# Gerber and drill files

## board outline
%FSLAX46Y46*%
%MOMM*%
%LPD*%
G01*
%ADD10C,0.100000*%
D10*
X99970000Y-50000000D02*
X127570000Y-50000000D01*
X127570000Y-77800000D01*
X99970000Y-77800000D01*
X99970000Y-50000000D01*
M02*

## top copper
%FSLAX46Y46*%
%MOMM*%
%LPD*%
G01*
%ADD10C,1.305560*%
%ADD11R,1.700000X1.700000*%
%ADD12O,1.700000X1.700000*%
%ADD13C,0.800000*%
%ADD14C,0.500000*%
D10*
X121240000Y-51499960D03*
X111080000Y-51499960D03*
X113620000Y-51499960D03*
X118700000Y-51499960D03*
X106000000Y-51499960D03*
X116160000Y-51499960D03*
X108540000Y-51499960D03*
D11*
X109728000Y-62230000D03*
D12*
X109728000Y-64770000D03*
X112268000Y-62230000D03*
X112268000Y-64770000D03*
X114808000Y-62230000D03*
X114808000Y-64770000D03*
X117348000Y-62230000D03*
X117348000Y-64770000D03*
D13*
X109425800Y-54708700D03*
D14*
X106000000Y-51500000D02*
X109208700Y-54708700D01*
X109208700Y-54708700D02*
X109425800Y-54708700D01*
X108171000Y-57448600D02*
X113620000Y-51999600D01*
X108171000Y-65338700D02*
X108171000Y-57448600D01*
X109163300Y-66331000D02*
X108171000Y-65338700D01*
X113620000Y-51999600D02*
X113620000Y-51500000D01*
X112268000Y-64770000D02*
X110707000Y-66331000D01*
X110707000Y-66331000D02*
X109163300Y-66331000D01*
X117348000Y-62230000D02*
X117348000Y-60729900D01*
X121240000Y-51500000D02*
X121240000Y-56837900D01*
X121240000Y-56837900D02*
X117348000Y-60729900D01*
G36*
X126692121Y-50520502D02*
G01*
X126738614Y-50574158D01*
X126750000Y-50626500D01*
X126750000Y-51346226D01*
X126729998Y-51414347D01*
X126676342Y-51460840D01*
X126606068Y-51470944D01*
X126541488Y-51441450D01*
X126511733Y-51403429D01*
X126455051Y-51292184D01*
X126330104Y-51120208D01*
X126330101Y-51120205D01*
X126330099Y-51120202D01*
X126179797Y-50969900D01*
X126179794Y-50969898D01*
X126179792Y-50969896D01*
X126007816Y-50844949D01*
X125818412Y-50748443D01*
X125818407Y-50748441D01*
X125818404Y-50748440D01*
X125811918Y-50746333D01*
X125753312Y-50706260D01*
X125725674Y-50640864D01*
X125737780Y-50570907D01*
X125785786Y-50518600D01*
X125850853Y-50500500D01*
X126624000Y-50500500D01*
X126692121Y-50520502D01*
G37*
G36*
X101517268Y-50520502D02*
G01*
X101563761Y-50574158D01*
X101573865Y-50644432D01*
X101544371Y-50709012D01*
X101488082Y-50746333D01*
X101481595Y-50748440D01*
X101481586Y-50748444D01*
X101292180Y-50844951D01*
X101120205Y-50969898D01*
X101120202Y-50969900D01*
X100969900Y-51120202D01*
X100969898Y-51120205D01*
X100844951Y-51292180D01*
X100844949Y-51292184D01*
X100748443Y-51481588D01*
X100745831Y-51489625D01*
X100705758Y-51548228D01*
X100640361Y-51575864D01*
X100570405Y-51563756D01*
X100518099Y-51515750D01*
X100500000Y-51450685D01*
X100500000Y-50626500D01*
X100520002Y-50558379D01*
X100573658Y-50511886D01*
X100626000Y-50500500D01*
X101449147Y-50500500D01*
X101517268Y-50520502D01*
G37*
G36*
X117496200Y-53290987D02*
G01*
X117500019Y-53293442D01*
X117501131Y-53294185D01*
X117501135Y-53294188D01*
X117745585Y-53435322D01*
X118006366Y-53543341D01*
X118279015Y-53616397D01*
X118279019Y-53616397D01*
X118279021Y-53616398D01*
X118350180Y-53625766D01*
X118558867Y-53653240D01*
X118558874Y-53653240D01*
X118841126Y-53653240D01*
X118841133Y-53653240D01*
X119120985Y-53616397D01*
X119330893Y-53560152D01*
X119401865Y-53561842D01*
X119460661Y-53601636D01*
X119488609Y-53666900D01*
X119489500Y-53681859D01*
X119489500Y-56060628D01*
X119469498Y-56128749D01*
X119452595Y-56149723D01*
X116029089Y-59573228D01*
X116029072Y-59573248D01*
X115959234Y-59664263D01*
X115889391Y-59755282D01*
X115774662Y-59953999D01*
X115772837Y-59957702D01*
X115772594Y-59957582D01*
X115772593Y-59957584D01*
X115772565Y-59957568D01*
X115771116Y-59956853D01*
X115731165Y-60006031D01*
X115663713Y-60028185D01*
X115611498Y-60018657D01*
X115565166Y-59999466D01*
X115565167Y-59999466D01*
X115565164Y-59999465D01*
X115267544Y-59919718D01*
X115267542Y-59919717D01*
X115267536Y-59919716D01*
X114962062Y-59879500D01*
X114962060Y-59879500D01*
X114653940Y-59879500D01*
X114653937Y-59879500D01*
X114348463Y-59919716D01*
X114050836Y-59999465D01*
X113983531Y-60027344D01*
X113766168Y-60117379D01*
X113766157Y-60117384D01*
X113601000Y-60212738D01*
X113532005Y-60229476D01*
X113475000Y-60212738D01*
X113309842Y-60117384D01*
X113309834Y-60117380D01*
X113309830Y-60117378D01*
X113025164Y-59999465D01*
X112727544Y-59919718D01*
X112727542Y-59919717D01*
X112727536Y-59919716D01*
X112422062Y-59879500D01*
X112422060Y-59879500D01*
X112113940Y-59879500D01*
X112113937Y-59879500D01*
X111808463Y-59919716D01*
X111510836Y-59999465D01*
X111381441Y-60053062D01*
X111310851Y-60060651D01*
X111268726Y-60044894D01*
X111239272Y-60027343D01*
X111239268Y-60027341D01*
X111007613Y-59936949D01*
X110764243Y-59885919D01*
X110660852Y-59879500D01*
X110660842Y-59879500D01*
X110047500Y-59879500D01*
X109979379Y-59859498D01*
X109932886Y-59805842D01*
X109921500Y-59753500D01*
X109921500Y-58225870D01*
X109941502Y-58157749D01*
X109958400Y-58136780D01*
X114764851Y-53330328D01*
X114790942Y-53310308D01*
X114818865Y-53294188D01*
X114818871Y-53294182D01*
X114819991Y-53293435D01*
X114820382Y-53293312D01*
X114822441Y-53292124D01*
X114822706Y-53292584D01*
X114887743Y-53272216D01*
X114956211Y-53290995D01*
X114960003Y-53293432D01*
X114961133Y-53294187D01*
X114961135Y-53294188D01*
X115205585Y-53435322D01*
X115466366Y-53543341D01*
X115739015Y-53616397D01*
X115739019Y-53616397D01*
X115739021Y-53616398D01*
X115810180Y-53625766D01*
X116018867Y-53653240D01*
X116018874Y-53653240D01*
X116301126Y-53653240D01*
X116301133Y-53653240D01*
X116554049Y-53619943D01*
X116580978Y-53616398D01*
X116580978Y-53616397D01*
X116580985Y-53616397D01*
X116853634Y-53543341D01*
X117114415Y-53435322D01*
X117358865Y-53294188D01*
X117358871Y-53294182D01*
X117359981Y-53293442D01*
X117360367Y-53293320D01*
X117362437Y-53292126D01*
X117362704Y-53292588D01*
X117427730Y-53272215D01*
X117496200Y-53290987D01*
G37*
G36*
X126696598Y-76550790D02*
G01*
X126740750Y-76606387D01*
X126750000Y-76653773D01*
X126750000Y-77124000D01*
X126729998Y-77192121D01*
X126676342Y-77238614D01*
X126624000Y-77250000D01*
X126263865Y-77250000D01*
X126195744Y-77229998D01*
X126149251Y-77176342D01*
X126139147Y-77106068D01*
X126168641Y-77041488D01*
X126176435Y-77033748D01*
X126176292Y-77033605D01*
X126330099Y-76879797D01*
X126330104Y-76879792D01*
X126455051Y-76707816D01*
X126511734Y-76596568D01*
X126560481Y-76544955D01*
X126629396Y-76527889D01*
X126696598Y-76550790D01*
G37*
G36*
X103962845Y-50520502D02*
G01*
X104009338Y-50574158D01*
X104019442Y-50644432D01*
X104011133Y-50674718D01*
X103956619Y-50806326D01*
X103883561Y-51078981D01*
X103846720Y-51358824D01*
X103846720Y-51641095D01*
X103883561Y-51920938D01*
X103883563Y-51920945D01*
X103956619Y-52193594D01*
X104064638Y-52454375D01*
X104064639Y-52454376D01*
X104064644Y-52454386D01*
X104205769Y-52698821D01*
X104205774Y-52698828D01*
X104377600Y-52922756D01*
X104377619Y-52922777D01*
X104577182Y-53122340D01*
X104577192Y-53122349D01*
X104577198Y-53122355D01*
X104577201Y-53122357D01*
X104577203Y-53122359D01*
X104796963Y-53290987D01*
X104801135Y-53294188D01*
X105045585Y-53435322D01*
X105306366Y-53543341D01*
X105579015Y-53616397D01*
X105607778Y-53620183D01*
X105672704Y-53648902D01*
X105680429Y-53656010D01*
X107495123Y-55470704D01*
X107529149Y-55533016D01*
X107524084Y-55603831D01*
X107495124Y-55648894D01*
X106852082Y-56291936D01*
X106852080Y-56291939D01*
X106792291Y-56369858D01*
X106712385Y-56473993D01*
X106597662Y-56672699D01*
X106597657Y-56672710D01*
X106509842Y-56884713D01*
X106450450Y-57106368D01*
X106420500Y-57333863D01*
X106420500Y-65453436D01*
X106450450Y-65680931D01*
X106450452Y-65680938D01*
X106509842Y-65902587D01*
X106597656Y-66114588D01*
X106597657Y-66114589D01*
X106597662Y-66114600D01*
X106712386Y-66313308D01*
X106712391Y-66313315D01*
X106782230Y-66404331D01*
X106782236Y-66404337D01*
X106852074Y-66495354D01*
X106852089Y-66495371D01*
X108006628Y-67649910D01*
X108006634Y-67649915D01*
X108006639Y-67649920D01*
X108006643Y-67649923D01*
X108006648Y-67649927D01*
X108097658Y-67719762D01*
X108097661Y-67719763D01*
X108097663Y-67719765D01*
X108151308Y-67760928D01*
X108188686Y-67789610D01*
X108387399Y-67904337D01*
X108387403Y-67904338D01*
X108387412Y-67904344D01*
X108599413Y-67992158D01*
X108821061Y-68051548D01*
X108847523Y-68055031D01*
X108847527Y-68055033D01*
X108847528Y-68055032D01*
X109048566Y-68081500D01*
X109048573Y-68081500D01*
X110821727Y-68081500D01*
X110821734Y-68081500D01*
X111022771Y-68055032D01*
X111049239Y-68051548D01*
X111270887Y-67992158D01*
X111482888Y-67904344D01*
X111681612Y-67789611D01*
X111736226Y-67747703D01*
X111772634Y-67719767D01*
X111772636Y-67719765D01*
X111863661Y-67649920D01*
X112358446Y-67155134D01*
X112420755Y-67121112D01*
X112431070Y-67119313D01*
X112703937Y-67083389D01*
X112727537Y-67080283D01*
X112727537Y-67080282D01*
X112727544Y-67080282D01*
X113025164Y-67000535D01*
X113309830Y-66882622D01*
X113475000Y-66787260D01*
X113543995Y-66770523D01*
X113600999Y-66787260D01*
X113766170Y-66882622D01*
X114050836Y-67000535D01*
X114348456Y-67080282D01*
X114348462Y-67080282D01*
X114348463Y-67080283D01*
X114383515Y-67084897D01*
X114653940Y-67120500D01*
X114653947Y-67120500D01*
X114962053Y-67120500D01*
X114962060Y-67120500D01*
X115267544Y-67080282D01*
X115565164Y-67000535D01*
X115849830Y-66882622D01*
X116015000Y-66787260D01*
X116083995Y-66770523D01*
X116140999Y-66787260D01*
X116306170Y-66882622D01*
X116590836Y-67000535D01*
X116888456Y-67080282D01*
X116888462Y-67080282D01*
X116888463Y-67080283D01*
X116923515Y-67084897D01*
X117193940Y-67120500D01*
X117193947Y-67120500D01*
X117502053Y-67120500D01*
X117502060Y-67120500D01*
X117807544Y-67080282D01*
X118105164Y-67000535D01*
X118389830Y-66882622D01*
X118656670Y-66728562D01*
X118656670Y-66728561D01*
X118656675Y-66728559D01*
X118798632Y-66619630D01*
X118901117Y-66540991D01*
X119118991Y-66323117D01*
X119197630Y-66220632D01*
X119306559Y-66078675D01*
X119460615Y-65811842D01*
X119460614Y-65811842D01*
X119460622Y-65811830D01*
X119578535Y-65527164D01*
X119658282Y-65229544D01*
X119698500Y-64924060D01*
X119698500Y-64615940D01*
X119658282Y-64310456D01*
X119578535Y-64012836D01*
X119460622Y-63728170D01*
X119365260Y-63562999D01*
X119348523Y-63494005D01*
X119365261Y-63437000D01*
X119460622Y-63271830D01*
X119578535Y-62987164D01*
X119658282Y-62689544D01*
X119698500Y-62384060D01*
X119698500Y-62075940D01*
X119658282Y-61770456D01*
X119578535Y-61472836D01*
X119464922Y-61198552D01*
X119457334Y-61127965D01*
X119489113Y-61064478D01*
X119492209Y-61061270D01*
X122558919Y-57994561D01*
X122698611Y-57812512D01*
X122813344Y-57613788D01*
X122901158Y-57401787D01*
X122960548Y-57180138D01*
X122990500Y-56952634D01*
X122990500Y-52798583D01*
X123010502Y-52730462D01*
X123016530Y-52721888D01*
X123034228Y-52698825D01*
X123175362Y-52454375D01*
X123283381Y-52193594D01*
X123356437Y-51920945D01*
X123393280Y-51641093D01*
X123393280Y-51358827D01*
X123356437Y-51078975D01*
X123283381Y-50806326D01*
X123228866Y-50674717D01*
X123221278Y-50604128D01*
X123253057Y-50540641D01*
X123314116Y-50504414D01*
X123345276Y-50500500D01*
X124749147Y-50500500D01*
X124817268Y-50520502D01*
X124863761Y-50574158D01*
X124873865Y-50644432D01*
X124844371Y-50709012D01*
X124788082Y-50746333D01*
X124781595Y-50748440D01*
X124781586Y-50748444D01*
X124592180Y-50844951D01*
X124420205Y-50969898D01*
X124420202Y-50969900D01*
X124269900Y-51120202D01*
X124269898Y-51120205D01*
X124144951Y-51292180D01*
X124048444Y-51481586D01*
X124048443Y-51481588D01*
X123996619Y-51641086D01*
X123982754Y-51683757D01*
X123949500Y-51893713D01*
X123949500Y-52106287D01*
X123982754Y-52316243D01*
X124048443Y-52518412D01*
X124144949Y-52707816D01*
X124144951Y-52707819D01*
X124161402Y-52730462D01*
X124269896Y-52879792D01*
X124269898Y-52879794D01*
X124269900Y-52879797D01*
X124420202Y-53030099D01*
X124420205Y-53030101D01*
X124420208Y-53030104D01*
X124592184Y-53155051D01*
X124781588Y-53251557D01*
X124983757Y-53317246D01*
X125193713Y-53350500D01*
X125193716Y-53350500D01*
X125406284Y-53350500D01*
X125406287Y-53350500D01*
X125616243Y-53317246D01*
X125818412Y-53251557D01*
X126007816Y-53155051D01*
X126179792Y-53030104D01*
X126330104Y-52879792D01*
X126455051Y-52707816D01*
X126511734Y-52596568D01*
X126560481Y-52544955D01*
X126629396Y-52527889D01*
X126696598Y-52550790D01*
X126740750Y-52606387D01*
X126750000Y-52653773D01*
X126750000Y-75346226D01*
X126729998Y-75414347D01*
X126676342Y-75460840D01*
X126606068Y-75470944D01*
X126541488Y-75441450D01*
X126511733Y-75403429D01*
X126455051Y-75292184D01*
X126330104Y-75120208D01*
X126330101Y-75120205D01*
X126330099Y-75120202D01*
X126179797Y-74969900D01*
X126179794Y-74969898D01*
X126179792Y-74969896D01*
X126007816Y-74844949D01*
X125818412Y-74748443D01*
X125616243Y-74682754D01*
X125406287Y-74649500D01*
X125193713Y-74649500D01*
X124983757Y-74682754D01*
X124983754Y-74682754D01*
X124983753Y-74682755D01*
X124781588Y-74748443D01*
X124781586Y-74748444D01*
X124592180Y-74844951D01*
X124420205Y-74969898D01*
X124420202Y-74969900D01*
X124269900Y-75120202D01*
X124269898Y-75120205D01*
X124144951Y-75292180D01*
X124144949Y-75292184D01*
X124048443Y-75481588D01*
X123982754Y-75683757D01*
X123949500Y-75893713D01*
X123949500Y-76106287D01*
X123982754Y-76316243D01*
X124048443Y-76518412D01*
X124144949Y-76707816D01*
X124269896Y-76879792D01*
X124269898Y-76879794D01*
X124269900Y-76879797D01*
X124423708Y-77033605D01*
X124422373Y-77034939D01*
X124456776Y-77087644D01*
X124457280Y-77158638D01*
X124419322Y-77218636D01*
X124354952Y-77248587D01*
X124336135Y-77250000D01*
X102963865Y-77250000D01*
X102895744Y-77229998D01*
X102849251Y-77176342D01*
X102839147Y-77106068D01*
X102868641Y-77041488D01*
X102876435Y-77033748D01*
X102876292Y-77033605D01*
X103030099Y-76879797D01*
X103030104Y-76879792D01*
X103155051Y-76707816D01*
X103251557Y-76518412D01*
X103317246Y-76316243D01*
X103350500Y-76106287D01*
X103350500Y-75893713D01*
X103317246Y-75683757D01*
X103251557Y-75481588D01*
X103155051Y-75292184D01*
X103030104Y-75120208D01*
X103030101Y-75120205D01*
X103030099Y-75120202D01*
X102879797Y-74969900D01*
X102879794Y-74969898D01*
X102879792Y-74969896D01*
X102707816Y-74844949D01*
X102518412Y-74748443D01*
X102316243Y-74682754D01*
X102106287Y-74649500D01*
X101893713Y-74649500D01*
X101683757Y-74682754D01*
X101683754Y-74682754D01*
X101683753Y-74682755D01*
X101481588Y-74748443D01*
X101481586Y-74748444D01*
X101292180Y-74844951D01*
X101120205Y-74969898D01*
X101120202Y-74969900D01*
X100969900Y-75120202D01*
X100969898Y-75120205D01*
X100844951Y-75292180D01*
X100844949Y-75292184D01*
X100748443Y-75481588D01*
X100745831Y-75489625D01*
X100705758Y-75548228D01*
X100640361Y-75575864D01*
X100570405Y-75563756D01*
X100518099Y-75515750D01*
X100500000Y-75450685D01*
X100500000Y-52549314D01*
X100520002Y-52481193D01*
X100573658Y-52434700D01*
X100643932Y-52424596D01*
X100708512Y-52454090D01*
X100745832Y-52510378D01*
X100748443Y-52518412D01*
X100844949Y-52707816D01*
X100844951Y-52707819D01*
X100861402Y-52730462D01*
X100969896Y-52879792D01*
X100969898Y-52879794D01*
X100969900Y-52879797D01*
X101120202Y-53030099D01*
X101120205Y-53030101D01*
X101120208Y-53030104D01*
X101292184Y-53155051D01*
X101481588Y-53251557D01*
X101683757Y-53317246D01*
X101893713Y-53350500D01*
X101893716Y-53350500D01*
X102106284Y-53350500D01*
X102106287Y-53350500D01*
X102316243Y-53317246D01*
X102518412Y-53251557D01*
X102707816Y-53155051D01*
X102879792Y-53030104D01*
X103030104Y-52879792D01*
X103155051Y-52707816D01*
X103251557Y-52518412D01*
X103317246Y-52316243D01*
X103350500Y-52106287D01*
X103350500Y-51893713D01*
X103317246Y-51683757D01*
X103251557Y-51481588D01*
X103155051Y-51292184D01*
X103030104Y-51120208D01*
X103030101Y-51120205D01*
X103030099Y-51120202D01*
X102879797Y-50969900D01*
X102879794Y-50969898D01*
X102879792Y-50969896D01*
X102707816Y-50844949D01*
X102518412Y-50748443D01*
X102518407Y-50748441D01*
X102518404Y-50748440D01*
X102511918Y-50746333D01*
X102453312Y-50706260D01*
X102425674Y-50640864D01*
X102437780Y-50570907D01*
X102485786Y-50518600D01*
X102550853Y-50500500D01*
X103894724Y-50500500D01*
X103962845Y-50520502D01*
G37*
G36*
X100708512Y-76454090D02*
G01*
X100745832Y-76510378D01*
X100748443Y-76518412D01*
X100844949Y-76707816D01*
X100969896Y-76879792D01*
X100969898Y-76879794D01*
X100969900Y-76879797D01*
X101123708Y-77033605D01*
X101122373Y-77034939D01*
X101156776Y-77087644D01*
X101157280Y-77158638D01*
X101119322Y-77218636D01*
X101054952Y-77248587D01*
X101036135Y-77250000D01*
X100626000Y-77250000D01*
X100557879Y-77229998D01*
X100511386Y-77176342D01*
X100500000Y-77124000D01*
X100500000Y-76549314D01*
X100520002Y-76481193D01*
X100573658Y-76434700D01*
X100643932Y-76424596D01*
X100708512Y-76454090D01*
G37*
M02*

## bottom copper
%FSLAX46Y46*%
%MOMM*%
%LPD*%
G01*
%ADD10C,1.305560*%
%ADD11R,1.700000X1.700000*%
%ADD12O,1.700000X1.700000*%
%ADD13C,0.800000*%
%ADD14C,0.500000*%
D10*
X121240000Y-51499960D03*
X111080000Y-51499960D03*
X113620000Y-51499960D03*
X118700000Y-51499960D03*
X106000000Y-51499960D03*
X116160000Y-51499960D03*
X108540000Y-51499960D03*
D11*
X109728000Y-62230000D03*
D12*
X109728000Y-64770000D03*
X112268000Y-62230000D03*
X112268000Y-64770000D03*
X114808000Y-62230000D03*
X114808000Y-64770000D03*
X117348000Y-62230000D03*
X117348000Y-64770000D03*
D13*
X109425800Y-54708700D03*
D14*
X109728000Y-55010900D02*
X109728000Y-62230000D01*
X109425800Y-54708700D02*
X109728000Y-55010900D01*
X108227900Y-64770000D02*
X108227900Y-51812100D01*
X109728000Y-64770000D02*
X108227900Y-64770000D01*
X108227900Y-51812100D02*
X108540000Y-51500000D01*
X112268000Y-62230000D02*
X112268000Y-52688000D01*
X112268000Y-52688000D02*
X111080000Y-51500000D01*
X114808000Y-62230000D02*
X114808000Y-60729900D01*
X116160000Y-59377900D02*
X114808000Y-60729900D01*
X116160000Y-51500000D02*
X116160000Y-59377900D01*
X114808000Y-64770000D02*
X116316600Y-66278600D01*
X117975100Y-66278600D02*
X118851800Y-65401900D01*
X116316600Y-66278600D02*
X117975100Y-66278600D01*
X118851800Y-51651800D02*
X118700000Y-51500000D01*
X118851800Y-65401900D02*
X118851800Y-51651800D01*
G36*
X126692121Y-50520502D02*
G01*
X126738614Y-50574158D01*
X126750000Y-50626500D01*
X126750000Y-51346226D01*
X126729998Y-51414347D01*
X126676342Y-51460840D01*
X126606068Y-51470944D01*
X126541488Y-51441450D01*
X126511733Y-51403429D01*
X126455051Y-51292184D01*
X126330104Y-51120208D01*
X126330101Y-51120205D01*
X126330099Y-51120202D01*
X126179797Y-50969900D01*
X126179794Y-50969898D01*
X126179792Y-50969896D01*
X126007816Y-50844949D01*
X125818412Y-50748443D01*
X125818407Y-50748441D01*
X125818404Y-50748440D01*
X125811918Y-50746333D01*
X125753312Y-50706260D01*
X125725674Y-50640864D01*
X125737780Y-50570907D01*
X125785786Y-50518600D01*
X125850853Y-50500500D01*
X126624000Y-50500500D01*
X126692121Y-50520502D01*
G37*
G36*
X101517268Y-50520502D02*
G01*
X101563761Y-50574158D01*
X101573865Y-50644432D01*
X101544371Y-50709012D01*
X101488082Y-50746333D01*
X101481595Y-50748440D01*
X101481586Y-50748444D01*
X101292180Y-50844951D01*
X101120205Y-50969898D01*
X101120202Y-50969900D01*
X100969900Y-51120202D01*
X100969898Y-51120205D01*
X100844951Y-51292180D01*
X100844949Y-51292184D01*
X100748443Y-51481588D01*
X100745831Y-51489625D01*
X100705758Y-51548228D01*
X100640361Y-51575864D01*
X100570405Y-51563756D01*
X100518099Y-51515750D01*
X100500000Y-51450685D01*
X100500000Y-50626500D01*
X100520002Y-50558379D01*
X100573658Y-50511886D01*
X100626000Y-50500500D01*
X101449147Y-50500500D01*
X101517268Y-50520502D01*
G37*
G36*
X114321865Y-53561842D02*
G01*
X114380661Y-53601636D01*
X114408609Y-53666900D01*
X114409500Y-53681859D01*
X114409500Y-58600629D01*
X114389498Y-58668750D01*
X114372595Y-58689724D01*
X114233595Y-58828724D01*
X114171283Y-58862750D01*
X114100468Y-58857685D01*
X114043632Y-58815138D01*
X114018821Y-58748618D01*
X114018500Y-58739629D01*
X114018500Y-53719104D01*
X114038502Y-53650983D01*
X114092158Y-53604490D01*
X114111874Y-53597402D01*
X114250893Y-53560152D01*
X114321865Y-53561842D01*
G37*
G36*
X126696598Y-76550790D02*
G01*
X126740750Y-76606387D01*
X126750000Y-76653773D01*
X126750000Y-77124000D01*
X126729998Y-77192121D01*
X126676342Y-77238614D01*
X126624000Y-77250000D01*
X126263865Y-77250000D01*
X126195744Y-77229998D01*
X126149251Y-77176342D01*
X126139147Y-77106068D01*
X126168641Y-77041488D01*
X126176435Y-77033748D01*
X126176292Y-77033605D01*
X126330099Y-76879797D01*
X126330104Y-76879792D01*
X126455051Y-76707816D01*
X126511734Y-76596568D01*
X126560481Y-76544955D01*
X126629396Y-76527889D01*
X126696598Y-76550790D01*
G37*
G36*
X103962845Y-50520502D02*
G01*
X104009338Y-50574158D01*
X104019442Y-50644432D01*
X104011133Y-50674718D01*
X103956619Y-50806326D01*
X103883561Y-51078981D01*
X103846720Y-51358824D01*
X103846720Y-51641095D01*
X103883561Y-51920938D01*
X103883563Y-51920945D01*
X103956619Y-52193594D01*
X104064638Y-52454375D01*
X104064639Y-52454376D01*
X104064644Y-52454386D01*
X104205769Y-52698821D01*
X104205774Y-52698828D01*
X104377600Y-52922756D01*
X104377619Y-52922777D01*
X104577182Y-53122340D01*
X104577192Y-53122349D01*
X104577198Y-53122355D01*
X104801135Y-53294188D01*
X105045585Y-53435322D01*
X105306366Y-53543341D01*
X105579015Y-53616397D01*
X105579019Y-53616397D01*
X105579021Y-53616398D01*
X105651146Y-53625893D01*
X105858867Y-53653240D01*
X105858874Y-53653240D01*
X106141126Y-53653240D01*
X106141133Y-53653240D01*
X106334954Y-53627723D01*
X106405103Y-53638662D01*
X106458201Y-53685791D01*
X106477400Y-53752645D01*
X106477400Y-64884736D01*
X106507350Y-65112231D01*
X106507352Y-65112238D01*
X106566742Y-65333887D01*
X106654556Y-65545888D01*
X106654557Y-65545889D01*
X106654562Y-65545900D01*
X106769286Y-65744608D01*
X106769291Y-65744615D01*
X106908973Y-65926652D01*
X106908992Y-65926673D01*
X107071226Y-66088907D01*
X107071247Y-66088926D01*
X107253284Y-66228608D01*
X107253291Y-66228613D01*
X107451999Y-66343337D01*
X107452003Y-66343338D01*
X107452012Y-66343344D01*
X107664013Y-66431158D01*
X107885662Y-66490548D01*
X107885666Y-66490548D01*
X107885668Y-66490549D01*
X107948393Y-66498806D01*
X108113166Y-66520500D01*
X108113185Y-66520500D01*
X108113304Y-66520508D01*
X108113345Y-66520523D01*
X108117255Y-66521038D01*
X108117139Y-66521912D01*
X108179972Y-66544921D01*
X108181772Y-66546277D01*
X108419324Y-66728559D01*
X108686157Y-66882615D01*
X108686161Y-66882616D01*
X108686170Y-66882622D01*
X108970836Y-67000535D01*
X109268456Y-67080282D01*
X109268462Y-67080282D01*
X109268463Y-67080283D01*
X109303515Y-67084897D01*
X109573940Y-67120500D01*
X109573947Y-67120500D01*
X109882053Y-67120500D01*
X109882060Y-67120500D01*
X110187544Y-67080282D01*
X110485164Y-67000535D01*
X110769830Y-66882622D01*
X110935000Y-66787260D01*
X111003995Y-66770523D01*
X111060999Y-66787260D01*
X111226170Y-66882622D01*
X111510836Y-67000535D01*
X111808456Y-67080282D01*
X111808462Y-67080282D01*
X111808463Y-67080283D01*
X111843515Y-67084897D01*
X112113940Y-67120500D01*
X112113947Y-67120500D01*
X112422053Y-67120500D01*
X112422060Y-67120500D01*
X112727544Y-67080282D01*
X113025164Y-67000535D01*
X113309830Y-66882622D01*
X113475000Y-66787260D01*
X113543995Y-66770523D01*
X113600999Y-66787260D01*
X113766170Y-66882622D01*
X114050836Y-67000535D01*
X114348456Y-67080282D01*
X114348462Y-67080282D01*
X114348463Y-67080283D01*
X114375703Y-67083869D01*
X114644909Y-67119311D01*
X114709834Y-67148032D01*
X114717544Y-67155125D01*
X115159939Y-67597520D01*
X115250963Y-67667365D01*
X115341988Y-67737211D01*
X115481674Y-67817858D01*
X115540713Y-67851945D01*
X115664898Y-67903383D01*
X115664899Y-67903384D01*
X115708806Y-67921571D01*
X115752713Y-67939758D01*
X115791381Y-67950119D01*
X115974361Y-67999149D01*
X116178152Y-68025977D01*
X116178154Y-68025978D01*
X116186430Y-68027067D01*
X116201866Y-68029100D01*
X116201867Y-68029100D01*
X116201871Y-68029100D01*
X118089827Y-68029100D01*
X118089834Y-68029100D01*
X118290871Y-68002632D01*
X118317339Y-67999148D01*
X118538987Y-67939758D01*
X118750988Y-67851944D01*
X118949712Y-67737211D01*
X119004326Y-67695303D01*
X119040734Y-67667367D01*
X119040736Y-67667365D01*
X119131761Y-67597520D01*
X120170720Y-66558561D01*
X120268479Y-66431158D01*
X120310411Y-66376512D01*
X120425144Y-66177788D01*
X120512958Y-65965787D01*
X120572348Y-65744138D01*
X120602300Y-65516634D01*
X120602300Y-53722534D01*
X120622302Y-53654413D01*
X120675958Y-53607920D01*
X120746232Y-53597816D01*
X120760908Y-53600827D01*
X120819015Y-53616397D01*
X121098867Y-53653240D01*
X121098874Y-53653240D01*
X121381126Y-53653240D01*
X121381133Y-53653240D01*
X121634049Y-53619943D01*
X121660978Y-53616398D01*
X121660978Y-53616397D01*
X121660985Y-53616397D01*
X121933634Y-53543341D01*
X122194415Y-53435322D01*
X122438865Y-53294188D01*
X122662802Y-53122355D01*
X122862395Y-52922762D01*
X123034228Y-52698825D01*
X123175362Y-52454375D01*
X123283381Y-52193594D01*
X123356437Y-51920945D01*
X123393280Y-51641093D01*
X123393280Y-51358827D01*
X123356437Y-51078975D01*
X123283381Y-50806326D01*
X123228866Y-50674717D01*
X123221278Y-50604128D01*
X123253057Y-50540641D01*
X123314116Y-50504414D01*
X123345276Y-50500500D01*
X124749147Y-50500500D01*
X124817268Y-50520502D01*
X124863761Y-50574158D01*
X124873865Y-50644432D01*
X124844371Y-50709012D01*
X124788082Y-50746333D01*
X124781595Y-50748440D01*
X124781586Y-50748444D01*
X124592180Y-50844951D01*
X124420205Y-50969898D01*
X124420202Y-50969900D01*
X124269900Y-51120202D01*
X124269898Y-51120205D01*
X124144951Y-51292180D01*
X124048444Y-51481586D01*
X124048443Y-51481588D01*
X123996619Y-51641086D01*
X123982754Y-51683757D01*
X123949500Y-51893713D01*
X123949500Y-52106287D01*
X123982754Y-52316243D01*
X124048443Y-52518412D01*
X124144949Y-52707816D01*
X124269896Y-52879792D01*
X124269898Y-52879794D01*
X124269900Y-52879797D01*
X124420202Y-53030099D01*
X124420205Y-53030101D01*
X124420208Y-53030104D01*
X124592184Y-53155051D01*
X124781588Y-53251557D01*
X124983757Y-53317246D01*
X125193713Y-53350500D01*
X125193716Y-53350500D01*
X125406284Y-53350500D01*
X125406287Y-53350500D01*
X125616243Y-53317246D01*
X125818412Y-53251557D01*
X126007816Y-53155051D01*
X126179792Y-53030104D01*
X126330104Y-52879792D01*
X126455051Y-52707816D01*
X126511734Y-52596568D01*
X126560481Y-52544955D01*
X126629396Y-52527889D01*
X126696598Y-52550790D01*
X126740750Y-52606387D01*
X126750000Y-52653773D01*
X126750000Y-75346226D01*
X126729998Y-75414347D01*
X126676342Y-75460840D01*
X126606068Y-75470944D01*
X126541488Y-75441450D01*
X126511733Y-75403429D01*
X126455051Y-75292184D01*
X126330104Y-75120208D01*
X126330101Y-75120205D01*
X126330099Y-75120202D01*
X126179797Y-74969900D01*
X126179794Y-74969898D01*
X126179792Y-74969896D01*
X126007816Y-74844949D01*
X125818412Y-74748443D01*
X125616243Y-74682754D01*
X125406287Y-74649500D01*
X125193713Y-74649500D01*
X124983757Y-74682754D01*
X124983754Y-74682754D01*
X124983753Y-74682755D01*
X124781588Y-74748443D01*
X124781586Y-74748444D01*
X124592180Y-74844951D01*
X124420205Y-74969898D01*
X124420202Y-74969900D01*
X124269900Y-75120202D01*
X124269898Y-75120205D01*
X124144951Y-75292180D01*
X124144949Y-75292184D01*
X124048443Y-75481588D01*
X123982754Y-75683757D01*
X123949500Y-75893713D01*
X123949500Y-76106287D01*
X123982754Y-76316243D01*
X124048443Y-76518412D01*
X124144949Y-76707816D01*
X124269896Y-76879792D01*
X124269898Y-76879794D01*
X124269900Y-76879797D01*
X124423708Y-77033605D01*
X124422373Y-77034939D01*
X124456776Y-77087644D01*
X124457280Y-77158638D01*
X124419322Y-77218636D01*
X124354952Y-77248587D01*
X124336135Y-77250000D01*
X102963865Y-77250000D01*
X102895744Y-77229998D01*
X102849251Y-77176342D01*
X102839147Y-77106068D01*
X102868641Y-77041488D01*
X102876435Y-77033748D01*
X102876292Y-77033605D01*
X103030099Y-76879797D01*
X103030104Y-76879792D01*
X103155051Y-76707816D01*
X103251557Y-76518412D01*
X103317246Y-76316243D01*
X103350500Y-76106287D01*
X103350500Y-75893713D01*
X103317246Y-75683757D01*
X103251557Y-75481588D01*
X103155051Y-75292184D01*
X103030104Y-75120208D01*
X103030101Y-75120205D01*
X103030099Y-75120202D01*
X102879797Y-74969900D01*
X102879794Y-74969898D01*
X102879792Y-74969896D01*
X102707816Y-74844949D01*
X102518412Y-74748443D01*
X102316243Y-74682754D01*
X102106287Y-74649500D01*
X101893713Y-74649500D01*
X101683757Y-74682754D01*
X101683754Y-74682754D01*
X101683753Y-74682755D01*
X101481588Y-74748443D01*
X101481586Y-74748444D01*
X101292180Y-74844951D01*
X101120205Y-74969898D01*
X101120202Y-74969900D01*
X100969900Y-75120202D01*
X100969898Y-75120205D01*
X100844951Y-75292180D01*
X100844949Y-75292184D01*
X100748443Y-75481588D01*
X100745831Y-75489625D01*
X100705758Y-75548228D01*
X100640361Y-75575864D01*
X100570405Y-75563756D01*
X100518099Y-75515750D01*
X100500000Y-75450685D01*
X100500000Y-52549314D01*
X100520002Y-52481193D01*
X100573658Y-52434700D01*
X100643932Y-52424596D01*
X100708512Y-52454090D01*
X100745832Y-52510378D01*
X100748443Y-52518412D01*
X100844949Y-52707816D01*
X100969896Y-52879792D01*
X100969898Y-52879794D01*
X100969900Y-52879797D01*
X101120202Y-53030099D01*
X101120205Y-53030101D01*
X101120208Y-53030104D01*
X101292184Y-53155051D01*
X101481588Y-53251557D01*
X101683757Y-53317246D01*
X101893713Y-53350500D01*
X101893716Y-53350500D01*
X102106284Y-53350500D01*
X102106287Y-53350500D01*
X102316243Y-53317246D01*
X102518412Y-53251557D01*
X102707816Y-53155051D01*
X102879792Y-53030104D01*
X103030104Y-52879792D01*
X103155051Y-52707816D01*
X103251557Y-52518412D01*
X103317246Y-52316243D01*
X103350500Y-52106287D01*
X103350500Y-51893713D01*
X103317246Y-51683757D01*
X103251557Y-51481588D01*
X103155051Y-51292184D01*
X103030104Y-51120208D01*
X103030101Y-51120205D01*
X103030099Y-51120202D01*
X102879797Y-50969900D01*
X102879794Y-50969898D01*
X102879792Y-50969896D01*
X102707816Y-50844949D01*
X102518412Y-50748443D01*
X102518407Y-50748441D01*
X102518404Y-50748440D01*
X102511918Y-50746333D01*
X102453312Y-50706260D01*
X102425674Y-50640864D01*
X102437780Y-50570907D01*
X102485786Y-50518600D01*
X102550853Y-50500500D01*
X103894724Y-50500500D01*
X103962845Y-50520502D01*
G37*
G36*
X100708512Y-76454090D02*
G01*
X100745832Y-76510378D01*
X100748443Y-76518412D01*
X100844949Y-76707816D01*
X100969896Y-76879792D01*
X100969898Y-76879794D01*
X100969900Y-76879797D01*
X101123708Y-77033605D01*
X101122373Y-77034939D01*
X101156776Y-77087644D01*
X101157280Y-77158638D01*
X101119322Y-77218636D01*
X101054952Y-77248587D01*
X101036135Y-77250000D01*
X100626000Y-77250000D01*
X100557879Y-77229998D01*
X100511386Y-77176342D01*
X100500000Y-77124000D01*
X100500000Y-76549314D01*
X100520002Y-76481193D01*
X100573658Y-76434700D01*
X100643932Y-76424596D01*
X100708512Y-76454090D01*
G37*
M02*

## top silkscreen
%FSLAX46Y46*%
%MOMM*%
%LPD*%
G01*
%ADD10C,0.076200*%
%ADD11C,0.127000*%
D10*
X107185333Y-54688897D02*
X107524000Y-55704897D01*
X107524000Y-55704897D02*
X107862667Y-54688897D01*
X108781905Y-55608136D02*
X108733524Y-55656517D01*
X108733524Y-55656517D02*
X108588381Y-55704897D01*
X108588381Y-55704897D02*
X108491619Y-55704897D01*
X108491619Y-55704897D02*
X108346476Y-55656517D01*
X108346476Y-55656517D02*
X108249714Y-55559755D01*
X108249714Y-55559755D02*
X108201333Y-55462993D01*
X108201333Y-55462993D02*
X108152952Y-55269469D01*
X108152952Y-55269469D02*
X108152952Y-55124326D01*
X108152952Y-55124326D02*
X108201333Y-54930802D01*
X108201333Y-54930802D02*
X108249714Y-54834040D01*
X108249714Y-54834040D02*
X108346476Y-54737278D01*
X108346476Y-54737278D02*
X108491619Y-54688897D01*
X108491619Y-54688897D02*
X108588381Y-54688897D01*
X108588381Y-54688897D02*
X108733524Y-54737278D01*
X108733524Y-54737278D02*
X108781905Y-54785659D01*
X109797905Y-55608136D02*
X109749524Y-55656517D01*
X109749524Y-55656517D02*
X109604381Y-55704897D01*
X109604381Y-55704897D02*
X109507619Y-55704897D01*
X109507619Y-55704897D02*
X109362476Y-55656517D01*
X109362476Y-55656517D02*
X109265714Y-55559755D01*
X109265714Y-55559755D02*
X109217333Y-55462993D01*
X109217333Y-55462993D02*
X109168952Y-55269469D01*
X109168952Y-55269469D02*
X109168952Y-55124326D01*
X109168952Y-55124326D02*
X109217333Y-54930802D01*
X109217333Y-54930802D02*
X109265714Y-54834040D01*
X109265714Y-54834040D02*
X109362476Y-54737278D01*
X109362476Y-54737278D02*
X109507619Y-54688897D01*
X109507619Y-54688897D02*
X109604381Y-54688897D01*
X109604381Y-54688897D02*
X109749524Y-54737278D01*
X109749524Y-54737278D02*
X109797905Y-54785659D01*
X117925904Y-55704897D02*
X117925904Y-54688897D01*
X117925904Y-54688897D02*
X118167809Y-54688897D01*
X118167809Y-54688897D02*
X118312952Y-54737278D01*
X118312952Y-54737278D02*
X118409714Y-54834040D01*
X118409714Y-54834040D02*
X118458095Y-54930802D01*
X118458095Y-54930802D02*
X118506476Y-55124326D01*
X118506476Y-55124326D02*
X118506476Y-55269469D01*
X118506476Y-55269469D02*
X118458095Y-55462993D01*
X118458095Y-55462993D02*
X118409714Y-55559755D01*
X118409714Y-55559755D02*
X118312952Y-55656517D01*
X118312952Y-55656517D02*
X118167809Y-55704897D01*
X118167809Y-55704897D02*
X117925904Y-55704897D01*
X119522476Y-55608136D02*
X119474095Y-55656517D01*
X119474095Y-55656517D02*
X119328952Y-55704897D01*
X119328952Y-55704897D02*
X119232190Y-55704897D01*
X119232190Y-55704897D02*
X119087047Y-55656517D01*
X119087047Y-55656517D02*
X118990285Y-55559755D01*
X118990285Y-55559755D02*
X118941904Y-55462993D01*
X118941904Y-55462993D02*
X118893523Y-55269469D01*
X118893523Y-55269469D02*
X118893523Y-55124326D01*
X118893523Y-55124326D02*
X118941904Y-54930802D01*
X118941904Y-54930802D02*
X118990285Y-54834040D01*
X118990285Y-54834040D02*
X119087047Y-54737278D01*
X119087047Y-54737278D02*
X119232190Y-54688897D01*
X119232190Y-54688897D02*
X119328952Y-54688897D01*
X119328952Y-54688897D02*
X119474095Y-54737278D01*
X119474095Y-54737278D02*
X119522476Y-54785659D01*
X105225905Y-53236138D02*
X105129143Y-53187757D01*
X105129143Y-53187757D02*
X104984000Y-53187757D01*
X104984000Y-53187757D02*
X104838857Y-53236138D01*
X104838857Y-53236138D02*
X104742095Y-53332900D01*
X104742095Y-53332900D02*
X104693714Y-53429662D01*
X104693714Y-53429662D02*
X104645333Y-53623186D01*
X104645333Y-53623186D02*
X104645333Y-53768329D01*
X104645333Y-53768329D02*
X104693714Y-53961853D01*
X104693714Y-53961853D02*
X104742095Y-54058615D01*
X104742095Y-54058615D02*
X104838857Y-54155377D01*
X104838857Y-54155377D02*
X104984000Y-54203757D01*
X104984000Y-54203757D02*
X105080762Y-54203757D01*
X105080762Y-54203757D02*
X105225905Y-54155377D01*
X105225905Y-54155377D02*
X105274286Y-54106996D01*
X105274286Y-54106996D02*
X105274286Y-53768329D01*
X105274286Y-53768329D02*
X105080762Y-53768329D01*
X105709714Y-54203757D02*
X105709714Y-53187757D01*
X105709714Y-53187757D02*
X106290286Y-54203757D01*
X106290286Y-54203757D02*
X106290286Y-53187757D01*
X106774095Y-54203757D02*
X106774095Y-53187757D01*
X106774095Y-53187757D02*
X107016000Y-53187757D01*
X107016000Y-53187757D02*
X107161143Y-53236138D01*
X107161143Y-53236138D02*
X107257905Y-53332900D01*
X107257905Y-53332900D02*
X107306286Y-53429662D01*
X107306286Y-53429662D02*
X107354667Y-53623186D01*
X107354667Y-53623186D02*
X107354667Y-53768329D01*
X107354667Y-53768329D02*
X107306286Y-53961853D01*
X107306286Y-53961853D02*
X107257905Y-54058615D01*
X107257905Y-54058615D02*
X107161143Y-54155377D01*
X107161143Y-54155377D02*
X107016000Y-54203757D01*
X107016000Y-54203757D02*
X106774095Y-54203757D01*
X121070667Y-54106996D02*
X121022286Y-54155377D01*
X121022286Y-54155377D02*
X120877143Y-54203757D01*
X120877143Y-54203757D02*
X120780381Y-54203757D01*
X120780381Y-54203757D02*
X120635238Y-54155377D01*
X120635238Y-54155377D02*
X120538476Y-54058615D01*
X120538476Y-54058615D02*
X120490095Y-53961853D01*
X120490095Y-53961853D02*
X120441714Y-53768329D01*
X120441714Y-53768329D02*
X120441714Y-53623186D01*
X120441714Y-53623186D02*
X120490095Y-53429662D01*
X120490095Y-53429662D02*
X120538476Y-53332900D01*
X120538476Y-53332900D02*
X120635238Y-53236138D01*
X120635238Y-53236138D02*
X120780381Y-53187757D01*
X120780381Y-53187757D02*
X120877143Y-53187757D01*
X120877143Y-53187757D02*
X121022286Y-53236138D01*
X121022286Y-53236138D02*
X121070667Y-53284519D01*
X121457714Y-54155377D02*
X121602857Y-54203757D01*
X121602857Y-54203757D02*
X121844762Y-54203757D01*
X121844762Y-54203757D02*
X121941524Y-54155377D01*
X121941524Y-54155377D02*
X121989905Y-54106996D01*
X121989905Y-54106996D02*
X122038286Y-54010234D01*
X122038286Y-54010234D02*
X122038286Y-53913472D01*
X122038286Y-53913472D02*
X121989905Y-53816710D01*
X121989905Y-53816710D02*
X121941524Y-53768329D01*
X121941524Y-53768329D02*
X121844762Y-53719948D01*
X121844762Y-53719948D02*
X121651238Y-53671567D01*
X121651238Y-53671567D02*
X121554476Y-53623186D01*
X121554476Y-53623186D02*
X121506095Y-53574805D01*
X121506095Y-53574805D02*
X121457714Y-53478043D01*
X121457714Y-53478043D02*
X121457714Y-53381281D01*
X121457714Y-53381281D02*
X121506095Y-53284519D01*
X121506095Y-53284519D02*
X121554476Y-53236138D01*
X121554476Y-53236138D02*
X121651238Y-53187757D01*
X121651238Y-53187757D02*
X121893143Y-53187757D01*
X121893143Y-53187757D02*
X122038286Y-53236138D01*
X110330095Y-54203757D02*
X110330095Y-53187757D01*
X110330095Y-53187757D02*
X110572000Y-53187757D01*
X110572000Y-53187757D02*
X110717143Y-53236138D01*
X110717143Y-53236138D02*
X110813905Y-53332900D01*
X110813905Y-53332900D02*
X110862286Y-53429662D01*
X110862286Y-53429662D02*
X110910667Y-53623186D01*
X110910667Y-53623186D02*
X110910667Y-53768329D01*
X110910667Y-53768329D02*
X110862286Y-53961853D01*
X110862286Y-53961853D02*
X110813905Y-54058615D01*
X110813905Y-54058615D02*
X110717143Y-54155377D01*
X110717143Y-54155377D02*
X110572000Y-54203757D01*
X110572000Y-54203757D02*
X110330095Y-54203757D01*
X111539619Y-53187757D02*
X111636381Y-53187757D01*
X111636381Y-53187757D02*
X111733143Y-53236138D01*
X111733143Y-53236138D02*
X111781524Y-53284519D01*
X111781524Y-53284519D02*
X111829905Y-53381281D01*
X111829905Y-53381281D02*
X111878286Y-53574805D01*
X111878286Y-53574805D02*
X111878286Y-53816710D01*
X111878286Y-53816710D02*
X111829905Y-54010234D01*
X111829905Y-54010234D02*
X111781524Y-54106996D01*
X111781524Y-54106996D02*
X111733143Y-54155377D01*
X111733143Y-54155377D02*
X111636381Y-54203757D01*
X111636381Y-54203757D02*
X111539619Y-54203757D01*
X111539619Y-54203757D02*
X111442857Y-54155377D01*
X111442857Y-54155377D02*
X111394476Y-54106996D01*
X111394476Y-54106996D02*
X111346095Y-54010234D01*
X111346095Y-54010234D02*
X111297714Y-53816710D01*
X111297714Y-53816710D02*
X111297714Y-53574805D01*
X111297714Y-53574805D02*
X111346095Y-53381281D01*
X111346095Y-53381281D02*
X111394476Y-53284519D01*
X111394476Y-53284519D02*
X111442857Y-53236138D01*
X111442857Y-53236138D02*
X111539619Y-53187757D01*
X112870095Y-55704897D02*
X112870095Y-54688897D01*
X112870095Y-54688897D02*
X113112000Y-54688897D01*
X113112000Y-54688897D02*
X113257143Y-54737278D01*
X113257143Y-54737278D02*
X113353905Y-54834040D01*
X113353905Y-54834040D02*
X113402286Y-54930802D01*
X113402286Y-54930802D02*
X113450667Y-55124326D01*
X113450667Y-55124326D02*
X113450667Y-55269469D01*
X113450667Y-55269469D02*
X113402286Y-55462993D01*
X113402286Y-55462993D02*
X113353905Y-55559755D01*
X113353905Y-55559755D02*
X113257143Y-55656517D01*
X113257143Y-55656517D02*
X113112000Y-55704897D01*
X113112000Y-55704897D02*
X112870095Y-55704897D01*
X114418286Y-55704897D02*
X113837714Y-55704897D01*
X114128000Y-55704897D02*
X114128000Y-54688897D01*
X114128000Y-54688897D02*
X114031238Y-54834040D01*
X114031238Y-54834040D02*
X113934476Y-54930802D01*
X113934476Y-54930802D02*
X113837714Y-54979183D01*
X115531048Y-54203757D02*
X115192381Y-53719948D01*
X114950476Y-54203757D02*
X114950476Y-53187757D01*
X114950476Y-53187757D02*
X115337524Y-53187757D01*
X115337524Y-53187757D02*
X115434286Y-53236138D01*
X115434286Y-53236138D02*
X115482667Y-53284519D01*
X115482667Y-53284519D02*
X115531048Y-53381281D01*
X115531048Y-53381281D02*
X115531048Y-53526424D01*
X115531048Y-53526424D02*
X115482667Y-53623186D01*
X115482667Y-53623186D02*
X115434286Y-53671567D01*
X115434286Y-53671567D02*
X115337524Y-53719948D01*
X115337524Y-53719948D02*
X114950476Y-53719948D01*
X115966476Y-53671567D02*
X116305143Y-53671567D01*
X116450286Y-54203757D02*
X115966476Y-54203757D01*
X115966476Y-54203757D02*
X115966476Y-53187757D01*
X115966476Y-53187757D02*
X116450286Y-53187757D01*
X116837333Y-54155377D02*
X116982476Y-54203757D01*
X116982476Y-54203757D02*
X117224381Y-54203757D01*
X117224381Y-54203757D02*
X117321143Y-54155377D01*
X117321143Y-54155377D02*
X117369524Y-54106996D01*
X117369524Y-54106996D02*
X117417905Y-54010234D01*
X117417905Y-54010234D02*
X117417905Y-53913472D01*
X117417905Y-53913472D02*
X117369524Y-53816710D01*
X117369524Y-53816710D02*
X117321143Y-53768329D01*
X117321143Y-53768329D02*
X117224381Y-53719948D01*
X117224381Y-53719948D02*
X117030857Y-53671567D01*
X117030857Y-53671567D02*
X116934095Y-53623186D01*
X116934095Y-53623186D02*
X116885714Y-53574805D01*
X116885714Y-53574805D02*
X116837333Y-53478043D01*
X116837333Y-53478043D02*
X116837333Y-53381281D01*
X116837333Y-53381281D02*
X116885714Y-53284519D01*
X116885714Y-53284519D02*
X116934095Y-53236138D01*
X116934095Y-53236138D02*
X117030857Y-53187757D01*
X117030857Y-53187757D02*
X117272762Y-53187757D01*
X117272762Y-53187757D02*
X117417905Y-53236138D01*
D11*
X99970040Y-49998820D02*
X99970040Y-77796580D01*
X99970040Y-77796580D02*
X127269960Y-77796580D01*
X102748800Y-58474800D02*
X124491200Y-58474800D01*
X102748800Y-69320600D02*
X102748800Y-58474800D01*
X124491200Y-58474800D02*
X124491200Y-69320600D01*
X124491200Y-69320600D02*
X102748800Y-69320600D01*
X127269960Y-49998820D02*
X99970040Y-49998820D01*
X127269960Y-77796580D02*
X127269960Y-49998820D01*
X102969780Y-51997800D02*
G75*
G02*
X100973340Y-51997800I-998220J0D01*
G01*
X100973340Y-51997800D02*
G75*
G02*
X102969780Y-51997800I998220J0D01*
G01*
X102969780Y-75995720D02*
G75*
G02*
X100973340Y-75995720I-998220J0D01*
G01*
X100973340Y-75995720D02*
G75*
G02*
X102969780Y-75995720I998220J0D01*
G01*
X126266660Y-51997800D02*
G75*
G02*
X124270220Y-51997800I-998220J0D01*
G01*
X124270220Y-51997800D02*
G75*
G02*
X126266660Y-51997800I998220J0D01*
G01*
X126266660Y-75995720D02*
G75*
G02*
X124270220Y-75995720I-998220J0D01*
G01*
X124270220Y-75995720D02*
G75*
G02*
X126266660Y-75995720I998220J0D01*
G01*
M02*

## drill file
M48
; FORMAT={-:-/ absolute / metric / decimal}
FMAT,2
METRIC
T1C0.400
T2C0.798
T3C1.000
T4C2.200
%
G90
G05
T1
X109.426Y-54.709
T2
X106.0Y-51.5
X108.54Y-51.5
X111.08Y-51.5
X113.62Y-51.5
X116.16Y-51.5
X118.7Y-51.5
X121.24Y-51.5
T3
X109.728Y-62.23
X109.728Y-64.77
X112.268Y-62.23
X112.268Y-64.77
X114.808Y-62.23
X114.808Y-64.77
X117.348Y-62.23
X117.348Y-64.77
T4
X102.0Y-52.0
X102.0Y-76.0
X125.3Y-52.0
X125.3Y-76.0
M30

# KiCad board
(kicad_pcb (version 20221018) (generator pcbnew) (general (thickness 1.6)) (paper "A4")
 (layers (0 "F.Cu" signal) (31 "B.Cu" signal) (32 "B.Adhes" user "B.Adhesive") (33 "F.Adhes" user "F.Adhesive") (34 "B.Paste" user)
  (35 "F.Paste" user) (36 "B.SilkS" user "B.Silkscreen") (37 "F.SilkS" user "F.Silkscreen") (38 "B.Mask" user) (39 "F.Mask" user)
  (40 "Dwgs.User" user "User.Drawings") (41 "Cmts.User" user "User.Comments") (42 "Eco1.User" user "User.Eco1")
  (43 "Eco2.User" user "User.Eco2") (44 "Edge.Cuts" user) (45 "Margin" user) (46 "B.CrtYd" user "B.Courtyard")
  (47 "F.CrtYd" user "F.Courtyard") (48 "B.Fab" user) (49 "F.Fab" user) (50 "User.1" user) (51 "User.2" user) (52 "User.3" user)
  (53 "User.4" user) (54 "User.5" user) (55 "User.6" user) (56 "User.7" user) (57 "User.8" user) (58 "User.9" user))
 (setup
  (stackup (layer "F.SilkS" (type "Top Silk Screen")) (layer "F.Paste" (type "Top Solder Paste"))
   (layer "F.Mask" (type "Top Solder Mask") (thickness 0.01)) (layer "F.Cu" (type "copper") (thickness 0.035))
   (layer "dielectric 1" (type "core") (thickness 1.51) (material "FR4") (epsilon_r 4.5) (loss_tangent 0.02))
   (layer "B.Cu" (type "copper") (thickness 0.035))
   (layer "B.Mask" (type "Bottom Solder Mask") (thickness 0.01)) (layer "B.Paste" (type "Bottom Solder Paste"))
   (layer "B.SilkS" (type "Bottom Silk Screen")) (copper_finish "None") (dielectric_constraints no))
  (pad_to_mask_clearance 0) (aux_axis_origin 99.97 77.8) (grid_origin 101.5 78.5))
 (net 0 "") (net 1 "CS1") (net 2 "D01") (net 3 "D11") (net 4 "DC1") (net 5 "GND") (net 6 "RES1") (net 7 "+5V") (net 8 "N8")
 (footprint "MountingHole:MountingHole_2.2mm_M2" (layer "F.Cu") (at 125.3 52)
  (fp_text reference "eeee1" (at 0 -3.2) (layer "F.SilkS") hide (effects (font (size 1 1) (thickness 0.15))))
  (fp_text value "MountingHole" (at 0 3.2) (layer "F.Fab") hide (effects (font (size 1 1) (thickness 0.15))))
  (pad "" np_thru_hole circle (at 0 0) (size 2.2 2.2) (drill 2.2) (layers "*.Cu" "*.Mask")))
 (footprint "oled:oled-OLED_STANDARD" (layer "F.Cu") (at 113.62 63.8977)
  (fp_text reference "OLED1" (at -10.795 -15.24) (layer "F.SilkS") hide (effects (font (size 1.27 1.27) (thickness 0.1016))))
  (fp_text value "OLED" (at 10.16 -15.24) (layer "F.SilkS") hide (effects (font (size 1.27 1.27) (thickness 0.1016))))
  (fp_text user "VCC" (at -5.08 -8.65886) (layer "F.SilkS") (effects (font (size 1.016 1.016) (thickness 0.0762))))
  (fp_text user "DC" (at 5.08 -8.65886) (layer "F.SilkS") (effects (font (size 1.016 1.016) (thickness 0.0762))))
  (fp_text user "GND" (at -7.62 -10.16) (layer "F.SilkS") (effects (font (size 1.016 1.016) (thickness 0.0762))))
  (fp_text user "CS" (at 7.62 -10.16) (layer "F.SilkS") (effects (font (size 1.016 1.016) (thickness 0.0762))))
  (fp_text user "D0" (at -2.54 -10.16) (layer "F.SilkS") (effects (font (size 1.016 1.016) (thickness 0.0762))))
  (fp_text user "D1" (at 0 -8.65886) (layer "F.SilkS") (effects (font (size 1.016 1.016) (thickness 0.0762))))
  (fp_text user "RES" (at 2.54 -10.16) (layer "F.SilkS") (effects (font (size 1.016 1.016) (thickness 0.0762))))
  (fp_line (start -13.64996 -13.89888) (end -13.64996 13.89888) (stroke (width 0.127) (type solid)) (layer "F.SilkS"))
  (fp_line (start -13.64996 13.89888) (end 13.64996 13.89888) (stroke (width 0.127) (type solid)) (layer "F.SilkS"))
  (fp_line (start -10.8712 -5.4229) (end 10.8712 -5.4229) (stroke (width 0.127) (type solid)) (layer "F.SilkS"))
  (fp_line (start -10.8712 5.4229) (end -10.8712 -5.4229) (stroke (width 0.127) (type solid)) (layer "F.SilkS"))
  (fp_line (start 10.8712 -5.4229) (end 10.8712 5.4229) (stroke (width 0.127) (type solid)) (layer "F.SilkS"))
  (fp_line (start 10.8712 5.4229) (end -10.8712 5.4229) (stroke (width 0.127) (type solid)) (layer "F.SilkS"))
  (fp_line (start 13.64996 -13.89888) (end -13.64996 -13.89888) (stroke (width 0.127) (type solid)) (layer "F.SilkS"))
  (fp_line (start 13.64996 13.89888) (end 13.64996 -13.89888) (stroke (width 0.127) (type solid)) (layer "F.SilkS"))
  (fp_circle (center -11.64844 -11.8999) (end -11.64844 -12.89812) (stroke (width 0.127) (type solid)) (fill none) (layer "F.SilkS"))
  (fp_circle (center -11.64844 12.09802) (end -11.64844 11.0998) (stroke (width 0.127) (type solid)) (fill none) (layer "F.SilkS"))
  (fp_circle (center 11.64844 -11.8999) (end 11.64844 -12.89812) (stroke (width 0.127) (type solid)) (fill none) (layer "F.SilkS"))
  (fp_circle (center 11.64844 12.09802) (end 11.64844 11.0998) (stroke (width 0.127) (type solid)) (fill none) (layer "F.SilkS"))
  (pad "CS" thru_hole circle (at 7.62 -12.39774) (size 1.30556 1.30556) (drill 0.79756) (layers "*.Cu" "*.Paste" "*.Mask") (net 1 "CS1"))
  (pad "D0" thru_hole circle (at -2.54 -12.39774) (size 1.30556 1.30556) (drill 0.79756) (layers "*.Cu" "*.Paste" "*.Mask") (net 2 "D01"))
  (pad "D1" thru_hole circle (at 0 -12.39774) (size 1.30556 1.30556) (drill 0.79756) (layers "*.Cu" "*.Paste" "*.Mask") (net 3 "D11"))
  (pad "DC" thru_hole circle (at 5.08 -12.39774) (size 1.30556 1.30556) (drill 0.79756) (layers "*.Cu" "*.Paste" "*.Mask") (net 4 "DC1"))
  (pad "GND" thru_hole circle (at -7.62 -12.39774) (size 1.30556 1.30556) (drill 0.79756) (layers "*.Cu" "*.Paste" "*.Mask") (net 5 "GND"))
  (pad "RES" thru_hole circle (at 2.54 -12.39774) (size 1.30556 1.30556) (drill 0.79756) (layers "*.Cu" "*.Paste" "*.Mask") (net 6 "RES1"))
  (pad "VCC" thru_hole circle (at -5.08 -12.39774) (size 1.30556 1.30556) (drill 0.79756) (layers "*.Cu" "*.Paste" "*.Mask") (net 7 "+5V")))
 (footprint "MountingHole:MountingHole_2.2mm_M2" (layer "F.Cu") (at 125.3 76)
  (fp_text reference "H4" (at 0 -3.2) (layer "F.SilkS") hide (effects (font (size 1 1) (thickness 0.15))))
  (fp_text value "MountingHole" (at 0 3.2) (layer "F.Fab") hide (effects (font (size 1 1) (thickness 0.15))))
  (pad "" np_thru_hole circle (at 0 0) (size 2.2 2.2) (drill 2.2) (layers "*.Cu" "*.Mask")))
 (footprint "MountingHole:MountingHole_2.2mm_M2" (layer "F.Cu") (at 102 76)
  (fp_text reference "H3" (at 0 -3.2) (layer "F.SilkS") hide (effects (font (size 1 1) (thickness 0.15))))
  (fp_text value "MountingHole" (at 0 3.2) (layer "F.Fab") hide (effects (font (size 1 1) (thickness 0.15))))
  (pad "" np_thru_hole circle (at 0 0) (size 2.2 2.2) (drill 2.2) (layers "*.Cu" "*.Mask")))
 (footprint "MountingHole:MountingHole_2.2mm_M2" (layer "F.Cu") (at 102 52)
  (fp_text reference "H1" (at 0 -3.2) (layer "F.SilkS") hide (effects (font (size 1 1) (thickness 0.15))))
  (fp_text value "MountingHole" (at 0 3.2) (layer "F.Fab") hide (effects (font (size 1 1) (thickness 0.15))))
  (pad "" np_thru_hole circle (at 0 0) (size 2.2 2.2) (drill 2.2) (layers "*.Cu" "*.Mask")))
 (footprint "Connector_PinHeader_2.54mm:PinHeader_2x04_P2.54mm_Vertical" (layer "B.Cu") (at 109.728 62.23 -90)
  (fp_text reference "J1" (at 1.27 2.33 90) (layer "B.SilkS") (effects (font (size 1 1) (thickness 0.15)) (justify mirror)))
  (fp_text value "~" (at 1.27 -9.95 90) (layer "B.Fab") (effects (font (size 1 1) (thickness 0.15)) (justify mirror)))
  (pad "1" thru_hole rect (at 0 0 270) (size 1.7 1.7) (drill 1) (layers "*.Cu" "*.Mask") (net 5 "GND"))
  (pad "2" thru_hole oval (at 2.54 0 270) (size 1.7 1.7) (drill 1) (layers "*.Cu" "*.Mask") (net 7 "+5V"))
  (pad "3" thru_hole oval (at 0 -2.54 270) (size 1.7 1.7) (drill 1) (layers "*.Cu" "*.Mask") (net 2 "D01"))
  (pad "4" thru_hole oval (at 2.54 -2.54 270) (size 1.7 1.7) (drill 1) (layers "*.Cu" "*.Mask") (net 3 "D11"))
  (pad "5" thru_hole oval (at 0 -5.08 270) (size 1.7 1.7) (drill 1) (layers "*.Cu" "*.Mask") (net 6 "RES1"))
  (pad "6" thru_hole oval (at 2.54 -5.08 270) (size 1.7 1.7) (drill 1) (layers "*.Cu" "*.Mask") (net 4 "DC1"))
  (pad "7" thru_hole oval (at 0 -7.62 270) (size 1.7 1.7) (drill 1) (layers "*.Cu" "*.Mask") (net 1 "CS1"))
  (pad "8" thru_hole oval (at 2.54 -7.62 270) (size 1.7 1.7) (drill 1) (layers "*.Cu" "*.Mask") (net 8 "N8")))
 (gr_rect (start 99.97 50) (end 127.57 77.8) (stroke (width 0.1) (type default)) (fill none) (layer "Edge.Cuts"))
 (segment (start 106 51.5) (end 109.2087 54.7087) (width 0.5) (layer "F.Cu") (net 5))
 (segment (start 109.2087 54.7087) (end 109.4258 54.7087) (width 0.5) (layer "F.Cu") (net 5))
 (via (at 109.4258 54.7087) (size 0.8) (drill 0.4) (layers "F.Cu" "B.Cu") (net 5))
 (segment (start 109.728 55.0109) (end 109.728 62.23) (width 0.5) (layer "B.Cu") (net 5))
 (segment (start 109.4258 54.7087) (end 109.728 55.0109) (width 0.5) (layer "B.Cu") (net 5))
 (segment (start 108.2279 64.77) (end 108.2279 51.8121) (width 0.5) (layer "B.Cu") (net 7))
 (segment (start 109.728 64.77) (end 108.2279 64.77) (width 0.5) (layer "B.Cu") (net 7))
 (segment (start 108.2279 51.8121) (end 108.54 51.5) (width 0.5) (layer "B.Cu") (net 7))
 (segment (start 112.268 62.23) (end 112.268 52.688) (width 0.5) (layer "B.Cu") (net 2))
 (segment (start 112.268 52.688) (end 111.08 51.5) (width 0.5) (layer "B.Cu") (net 2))
 (segment (start 108.171 57.4486) (end 113.62 51.9996) (width 0.5) (layer "F.Cu") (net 3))
 (segment (start 108.171 65.3387) (end 108.171 57.4486) (width 0.5) (layer "F.Cu") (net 3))
 (segment (start 109.1633 66.331) (end 108.171 65.3387) (width 0.5) (layer "F.Cu") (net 3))
 (segment (start 113.62 51.9996) (end 113.62 51.5) (width 0.5) (layer "F.Cu") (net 3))
 (segment (start 112.268 64.77) (end 110.707 66.331) (width 0.5) (layer "F.Cu") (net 3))
 (segment (start 110.707 66.331) (end 109.1633 66.331) (width 0.5) (layer "F.Cu") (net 3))
 (segment (start 114.808 62.23) (end 114.808 60.7299) (width 0.5) (layer "B.Cu") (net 6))
 (segment (start 116.16 59.3779) (end 114.808 60.7299) (width 0.5) (layer "B.Cu") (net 6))
 (segment (start 116.16 51.5) (end 116.16 59.3779) (width 0.5) (layer "B.Cu") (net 6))
 (segment (start 114.808 64.77) (end 116.3166 66.2786) (width 0.5) (layer "B.Cu") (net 4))
 (segment (start 117.9751 66.2786) (end 118.8518 65.4019) (width 0.5) (layer "B.Cu") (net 4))
 (segment (start 116.3166 66.2786) (end 117.9751 66.2786) (width 0.5) (layer "B.Cu") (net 4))
 (segment (start 118.8518 51.6518) (end 118.7 51.5) (width 0.5) (layer "B.Cu") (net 4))
 (segment (start 118.8518 65.4019) (end 118.8518 51.6518) (width 0.5) (layer "B.Cu") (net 4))
 (segment (start 117.348 62.23) (end 117.348 60.7299) (width 0.5) (layer "F.Cu") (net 1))
 (segment (start 121.24 51.5) (end 121.24 56.8379) (width 0.5) (layer "F.Cu") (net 1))
 (segment (start 121.24 56.8379) (end 117.348 60.7299) (width 0.5) (layer "F.Cu") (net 1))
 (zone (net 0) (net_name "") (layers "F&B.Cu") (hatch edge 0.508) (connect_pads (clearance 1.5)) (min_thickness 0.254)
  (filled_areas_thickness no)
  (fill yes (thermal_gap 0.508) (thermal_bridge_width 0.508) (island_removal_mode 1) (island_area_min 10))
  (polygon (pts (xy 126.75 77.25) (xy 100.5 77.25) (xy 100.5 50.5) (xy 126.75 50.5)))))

